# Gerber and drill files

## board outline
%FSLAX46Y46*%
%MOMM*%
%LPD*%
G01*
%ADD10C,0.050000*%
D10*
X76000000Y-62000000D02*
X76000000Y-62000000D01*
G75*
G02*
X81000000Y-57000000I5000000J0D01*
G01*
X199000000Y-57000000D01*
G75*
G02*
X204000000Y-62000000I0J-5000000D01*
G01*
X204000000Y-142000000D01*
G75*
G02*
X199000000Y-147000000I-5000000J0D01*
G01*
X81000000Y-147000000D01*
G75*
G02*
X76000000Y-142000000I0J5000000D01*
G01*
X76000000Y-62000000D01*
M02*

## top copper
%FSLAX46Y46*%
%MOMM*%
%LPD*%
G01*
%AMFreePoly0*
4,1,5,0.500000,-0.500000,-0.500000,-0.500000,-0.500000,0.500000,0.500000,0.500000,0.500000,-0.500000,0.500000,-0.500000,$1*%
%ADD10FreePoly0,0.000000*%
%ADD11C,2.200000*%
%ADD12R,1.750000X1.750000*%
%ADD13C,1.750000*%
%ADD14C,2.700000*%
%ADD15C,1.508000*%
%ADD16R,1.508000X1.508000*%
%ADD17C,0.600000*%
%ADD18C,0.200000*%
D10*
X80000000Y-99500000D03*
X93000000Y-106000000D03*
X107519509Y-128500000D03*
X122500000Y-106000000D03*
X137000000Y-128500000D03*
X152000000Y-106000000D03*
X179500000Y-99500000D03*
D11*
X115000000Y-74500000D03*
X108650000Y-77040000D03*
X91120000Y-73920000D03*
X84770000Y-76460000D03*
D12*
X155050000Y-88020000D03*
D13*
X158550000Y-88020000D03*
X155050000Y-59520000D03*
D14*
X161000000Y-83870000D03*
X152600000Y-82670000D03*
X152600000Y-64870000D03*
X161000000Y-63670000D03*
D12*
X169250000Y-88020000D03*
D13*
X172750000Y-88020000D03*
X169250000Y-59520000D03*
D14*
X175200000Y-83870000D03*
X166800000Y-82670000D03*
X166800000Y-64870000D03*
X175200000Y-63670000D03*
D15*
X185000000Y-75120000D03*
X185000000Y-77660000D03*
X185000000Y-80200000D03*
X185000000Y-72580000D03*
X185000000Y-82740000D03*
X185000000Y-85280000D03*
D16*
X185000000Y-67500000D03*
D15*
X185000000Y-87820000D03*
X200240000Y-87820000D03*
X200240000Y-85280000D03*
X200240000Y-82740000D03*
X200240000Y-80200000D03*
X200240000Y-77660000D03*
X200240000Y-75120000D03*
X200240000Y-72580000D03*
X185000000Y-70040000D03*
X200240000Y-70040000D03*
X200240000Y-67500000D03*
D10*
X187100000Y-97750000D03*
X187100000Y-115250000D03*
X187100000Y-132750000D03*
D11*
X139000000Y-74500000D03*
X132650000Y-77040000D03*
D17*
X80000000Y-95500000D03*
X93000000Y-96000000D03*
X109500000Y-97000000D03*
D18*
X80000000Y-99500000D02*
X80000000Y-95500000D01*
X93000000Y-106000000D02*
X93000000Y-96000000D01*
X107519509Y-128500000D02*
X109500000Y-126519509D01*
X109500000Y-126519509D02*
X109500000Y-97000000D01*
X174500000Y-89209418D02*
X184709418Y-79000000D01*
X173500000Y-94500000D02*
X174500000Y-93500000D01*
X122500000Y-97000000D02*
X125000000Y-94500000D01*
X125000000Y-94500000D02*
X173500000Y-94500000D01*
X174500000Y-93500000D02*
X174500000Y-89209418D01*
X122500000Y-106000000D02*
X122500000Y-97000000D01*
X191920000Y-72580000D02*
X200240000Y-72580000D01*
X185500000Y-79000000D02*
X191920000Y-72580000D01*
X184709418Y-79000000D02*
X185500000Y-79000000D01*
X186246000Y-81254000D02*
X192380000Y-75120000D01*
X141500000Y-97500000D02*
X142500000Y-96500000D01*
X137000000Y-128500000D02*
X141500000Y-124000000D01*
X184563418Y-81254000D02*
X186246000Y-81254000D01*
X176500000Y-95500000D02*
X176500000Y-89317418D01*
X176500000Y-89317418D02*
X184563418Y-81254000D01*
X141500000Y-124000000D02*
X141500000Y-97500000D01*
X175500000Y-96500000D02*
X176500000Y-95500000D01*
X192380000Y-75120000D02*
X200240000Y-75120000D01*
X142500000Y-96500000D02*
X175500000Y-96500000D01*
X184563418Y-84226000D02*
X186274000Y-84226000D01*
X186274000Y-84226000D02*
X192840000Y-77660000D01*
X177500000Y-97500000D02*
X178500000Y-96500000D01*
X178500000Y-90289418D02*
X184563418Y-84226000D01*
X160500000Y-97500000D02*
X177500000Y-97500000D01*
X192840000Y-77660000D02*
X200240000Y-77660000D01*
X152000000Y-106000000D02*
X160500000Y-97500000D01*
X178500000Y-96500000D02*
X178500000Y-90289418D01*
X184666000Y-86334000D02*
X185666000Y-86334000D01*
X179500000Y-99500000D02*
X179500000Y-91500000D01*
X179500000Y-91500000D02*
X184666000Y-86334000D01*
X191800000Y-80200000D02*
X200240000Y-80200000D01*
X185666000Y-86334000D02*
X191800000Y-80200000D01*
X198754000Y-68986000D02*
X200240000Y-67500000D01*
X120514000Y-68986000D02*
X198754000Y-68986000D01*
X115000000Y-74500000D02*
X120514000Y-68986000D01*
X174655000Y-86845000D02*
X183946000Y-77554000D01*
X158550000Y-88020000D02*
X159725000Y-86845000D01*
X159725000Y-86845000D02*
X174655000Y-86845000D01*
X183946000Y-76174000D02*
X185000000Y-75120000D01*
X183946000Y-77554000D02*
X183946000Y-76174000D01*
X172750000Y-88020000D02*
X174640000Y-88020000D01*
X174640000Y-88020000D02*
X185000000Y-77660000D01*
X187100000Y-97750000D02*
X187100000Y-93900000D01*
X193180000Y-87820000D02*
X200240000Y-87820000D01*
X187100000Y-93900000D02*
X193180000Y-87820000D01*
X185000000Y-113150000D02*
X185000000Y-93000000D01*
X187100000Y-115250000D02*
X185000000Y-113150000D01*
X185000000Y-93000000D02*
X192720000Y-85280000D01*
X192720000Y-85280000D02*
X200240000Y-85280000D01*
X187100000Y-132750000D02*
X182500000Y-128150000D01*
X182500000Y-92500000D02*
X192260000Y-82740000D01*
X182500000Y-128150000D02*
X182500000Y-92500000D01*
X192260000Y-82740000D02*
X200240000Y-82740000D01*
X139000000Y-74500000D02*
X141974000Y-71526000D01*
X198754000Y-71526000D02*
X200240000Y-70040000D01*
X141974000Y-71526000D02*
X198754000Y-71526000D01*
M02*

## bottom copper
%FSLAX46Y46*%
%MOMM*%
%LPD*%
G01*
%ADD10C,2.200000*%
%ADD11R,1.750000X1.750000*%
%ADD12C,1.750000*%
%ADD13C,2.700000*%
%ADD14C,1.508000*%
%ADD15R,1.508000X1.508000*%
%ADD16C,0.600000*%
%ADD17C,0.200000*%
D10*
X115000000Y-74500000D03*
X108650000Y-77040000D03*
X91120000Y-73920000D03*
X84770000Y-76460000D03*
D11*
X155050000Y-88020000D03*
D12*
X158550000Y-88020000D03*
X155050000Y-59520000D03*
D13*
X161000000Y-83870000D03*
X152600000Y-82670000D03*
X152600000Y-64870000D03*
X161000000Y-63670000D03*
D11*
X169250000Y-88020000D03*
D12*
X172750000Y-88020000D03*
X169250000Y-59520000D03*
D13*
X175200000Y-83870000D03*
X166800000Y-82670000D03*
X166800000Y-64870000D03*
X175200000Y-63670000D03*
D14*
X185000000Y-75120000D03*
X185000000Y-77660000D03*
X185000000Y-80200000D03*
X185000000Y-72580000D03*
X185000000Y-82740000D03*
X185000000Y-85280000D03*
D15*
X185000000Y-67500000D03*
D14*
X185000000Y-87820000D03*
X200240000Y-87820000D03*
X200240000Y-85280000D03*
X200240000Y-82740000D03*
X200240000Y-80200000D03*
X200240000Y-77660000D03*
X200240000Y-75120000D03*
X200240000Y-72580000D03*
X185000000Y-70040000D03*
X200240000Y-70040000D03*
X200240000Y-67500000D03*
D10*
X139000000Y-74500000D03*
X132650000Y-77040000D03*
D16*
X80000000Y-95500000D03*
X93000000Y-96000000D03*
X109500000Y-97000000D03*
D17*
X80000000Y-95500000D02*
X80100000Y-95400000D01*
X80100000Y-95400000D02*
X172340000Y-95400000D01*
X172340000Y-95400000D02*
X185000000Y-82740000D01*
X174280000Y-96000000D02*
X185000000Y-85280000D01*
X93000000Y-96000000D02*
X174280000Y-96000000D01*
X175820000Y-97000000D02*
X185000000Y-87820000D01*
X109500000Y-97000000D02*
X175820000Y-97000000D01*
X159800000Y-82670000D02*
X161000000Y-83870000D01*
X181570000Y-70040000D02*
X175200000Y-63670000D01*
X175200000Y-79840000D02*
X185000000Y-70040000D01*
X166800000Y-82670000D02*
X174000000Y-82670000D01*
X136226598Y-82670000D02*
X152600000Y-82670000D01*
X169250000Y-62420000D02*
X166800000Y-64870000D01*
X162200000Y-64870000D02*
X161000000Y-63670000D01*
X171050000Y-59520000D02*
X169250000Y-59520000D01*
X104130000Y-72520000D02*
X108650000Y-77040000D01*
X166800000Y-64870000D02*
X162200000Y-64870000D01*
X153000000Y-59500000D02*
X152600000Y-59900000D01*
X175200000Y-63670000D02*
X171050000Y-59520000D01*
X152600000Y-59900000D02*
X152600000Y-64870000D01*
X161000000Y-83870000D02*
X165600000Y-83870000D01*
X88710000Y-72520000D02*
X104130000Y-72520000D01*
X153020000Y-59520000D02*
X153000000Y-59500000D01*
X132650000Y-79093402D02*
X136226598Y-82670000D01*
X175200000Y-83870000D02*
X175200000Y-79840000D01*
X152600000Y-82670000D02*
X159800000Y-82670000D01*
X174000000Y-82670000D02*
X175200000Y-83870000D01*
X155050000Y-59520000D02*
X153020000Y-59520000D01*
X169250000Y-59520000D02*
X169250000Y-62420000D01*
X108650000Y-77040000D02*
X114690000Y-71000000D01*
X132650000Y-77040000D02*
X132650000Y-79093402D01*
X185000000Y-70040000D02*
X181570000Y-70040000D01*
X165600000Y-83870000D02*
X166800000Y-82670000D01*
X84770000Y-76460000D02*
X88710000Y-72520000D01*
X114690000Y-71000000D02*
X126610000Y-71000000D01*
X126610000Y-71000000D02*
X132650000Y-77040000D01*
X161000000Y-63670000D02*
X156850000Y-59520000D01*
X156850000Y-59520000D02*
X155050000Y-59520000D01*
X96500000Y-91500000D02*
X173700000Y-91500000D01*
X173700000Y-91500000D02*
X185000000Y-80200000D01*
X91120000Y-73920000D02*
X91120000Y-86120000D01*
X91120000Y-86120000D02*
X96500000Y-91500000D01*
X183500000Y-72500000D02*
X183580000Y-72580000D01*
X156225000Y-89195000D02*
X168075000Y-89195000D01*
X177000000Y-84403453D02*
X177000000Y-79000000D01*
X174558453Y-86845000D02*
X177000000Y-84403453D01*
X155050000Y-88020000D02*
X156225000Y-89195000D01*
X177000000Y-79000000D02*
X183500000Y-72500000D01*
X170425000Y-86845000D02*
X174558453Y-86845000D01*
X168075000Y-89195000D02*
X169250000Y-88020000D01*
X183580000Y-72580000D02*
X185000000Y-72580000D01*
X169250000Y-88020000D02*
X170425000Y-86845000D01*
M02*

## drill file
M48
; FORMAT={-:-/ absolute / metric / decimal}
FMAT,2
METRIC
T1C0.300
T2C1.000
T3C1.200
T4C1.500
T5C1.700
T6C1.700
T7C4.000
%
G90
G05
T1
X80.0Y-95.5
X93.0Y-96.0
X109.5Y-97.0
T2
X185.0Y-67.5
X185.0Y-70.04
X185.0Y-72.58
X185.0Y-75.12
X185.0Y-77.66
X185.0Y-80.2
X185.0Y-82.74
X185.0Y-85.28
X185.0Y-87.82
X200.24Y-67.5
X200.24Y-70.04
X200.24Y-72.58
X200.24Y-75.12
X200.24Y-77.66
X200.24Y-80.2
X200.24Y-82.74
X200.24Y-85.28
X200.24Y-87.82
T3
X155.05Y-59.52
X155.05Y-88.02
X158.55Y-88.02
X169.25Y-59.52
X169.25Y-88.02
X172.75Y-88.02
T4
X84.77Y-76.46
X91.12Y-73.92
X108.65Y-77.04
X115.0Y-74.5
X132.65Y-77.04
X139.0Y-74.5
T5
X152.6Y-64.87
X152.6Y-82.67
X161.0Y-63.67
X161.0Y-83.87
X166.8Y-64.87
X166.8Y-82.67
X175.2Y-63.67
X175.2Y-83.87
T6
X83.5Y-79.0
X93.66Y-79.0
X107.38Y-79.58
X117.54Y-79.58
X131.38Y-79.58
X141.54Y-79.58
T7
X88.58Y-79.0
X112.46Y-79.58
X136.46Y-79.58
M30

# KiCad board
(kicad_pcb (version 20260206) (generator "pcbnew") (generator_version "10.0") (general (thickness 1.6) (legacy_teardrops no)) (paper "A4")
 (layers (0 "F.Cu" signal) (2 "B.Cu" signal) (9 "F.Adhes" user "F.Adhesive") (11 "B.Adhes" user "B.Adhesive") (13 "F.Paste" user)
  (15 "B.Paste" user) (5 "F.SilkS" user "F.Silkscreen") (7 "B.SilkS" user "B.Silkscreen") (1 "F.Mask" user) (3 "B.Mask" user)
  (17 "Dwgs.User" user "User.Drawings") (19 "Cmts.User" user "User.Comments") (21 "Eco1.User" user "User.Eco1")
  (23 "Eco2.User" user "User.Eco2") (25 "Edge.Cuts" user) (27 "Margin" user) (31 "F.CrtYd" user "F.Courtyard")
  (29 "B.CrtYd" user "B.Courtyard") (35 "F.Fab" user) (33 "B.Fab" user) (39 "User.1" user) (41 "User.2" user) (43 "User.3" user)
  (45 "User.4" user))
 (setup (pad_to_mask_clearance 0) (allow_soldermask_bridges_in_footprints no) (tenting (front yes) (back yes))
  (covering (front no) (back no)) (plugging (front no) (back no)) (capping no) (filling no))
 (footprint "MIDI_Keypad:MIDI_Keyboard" (layer "F.Cu") (at 104 43)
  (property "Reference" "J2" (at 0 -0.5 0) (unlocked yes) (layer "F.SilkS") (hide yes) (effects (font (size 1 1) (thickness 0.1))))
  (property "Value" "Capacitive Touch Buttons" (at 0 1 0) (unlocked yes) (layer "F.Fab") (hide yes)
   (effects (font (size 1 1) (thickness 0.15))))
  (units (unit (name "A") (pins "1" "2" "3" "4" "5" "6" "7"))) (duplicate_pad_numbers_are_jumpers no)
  (pad "1" smd custom (at -24 56.5) (size 1 1) (layers "F.Cu" "F.Mask") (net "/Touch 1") (options (clearance outline) (anchor rect))
   (primitives))
  (pad "2" smd custom (at -11 63) (size 1 1) (layers "F.Cu" "F.Mask") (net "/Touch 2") (options (clearance outline) (anchor rect))
   (primitives))
  (pad "3" smd custom (at 3.519509 85.5) (size 1 1) (layers "F.Cu" "F.Mask") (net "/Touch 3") (options (clearance outline) (anchor rect))
   (primitives))
  (pad "4" smd custom (at 18.5 63) (size 1 1) (layers "F.Cu" "F.Mask") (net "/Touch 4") (options (clearance outline) (anchor rect))
   (primitives))
  (pad "5" smd custom (at 33 85.5) (size 1 1) (layers "F.Cu" "F.Mask") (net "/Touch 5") (options (clearance outline) (anchor rect))
   (primitives))
  (pad "6" smd custom (at 48 63) (size 1 1) (layers "F.Cu" "F.Mask") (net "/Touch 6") (options (clearance outline) (anchor rect))
   (primitives))
  (pad "7" smd custom (at 75.5 56.5) (size 1 1) (layers "F.Cu" "F.Mask") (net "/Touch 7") (options (clearance outline) (anchor rect))
   (primitives)))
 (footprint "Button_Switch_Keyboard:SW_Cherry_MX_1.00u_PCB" (layer "F.Cu") (at 115 74.5)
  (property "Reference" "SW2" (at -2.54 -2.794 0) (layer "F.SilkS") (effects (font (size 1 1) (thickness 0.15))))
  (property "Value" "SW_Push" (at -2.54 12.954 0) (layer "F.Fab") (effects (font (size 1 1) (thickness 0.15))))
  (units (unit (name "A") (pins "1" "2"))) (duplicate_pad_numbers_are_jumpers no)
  (pad "" np_thru_hole circle (at -7.62 5.08) (size 1.7 1.7) (drill 1.7) (layers "*.Cu" "*.Mask"))
  (pad "" np_thru_hole circle (at -2.54 5.08) (size 4 4) (drill 4) (layers "*.Cu" "*.Mask"))
  (pad "" np_thru_hole circle (at 2.54 5.08) (size 1.7 1.7) (drill 1.7) (layers "*.Cu" "*.Mask"))
  (pad "1" thru_hole circle (at 0 0) (size 2.2 2.2) (drill 1.5) (layers "*.Cu" "*.Mask") (remove_unused_layers no) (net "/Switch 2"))
  (pad "2" thru_hole circle (at -6.35 2.54) (size 2.2 2.2) (drill 1.5) (layers "*.Cu" "*.Mask") (remove_unused_layers no) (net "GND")))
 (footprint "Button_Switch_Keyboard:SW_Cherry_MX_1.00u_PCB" (layer "F.Cu") (at 91.12 73.92)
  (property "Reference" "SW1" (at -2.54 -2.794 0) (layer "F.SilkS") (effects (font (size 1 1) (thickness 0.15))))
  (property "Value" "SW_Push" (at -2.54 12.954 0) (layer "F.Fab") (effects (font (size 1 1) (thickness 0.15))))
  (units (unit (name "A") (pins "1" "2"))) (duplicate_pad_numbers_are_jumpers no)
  (pad "" np_thru_hole circle (at -7.62 5.08) (size 1.7 1.7) (drill 1.7) (layers "*.Cu" "*.Mask"))
  (pad "" np_thru_hole circle (at -2.54 5.08) (size 4 4) (drill 4) (layers "*.Cu" "*.Mask"))
  (pad "" np_thru_hole circle (at 2.54 5.08) (size 1.7 1.7) (drill 1.7) (layers "*.Cu" "*.Mask"))
  (pad "1" thru_hole circle (at 0 0) (size 2.2 2.2) (drill 1.5) (layers "*.Cu" "*.Mask") (remove_unused_layers no) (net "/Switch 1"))
  (pad "2" thru_hole circle (at -6.35 2.54) (size 2.2 2.2) (drill 1.5) (layers "*.Cu" "*.Mask") (remove_unused_layers no) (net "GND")))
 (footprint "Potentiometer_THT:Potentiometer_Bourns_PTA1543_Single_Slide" (layer "F.Cu") (at 155.05 88.02 90)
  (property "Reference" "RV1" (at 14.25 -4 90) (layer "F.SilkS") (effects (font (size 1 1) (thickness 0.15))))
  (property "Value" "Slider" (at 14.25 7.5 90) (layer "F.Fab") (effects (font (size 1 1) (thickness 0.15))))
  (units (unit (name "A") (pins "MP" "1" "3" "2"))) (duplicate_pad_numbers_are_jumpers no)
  (pad "1" thru_hole rect (at 0 0 90) (size 1.75 1.75) (drill 1.2) (layers "*.Cu" "*.Mask") (remove_unused_layers no) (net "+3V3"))
  (pad "2" thru_hole circle (at 0 3.5 90) (size 1.75 1.75) (drill 1.2) (layers "*.Cu" "*.Mask") (remove_unused_layers no) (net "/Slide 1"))
  (pad "3" thru_hole circle (at 28.5 0 90) (size 1.75 1.75) (drill 1.2) (layers "*.Cu" "*.Mask") (remove_unused_layers no) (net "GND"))
  (pad "MP" thru_hole circle (at 4.15 5.95 90) (size 2.7 2.7) (drill 1.7) (layers "*.Cu" "*.Mask") (remove_unused_layers no) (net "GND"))
  (pad "MP" thru_hole circle (at 5.35 -2.45 90) (size 2.7 2.7) (drill 1.7) (layers "*.Cu" "*.Mask") (remove_unused_layers no) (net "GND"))
  (pad "MP" thru_hole circle (at 23.15 -2.45 90) (size 2.7 2.7) (drill 1.7) (layers "*.Cu" "*.Mask") (remove_unused_layers no) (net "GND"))
  (pad "MP" thru_hole circle (at 24.35 5.95 90) (size 2.7 2.7) (drill 1.7) (layers "*.Cu" "*.Mask") (remove_unused_layers no) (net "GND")))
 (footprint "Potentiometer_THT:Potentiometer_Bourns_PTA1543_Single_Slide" (layer "F.Cu") (at 169.25 88.02 90)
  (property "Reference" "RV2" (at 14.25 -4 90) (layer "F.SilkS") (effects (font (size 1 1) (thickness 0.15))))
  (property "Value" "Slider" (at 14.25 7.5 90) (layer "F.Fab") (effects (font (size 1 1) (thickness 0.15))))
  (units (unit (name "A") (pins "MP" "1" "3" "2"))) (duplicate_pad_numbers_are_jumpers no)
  (pad "1" thru_hole rect (at 0 0 90) (size 1.75 1.75) (drill 1.2) (layers "*.Cu" "*.Mask") (remove_unused_layers no) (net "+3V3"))
  (pad "2" thru_hole circle (at 0 3.5 90) (size 1.75 1.75) (drill 1.2) (layers "*.Cu" "*.Mask") (remove_unused_layers no) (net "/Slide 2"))
  (pad "3" thru_hole circle (at 28.5 0 90) (size 1.75 1.75) (drill 1.2) (layers "*.Cu" "*.Mask") (remove_unused_layers no) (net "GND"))
  (pad "MP" thru_hole circle (at 4.15 5.95 90) (size 2.7 2.7) (drill 1.7) (layers "*.Cu" "*.Mask") (remove_unused_layers no) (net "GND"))
  (pad "MP" thru_hole circle (at 5.35 -2.45 90) (size 2.7 2.7) (drill 1.7) (layers "*.Cu" "*.Mask") (remove_unused_layers no) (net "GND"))
  (pad "MP" thru_hole circle (at 23.15 -2.45 90) (size 2.7 2.7) (drill 1.7) (layers "*.Cu" "*.Mask") (remove_unused_layers no) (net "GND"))
  (pad "MP" thru_hole circle (at 24.35 5.95 90) (size 2.7 2.7) (drill 1.7) (layers "*.Cu" "*.Mask") (remove_unused_layers no) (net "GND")))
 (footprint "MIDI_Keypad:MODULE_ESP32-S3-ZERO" (layer "F.Cu") (at 192.62 77.66)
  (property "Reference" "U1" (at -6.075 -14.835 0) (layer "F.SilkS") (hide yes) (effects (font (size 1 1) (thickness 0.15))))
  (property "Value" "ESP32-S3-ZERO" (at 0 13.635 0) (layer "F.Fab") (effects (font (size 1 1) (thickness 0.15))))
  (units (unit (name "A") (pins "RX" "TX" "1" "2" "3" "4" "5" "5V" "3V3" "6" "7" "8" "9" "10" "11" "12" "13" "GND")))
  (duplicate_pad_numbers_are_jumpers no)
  (pad "1" thru_hole circle (at -7.62 -2.54) (size 1.508 1.508) (drill 1) (layers "*.Cu" "*.Mask") (remove_unused_layers no)
   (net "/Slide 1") (solder_mask_margin 0.102))
  (pad "2" thru_hole circle (at -7.62 0) (size 1.508 1.508) (drill 1) (layers "*.Cu" "*.Mask") (remove_unused_layers no) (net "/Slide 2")
   (solder_mask_margin 0.102))
  (pad "3" thru_hole circle (at -7.62 2.54) (size 1.508 1.508) (drill 1) (layers "*.Cu" "*.Mask") (remove_unused_layers no)
   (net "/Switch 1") (solder_mask_margin 0.102))
  (pad "3V3" thru_hole circle (at -7.62 -5.08) (size 1.508 1.508) (drill 1) (layers "*.Cu" "*.Mask") (remove_unused_layers no) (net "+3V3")
   (solder_mask_margin 0.102))
  (pad "4" thru_hole circle (at -7.62 5.08) (size 1.508 1.508) (drill 1) (layers "*.Cu" "*.Mask") (remove_unused_layers no) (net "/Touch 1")
   (solder_mask_margin 0.102))
  (pad "5" thru_hole circle (at -7.62 7.62) (size 1.508 1.508) (drill 1) (layers "*.Cu" "*.Mask") (remove_unused_layers no) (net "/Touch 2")
   (solder_mask_margin 0.102))
  (pad "5V" thru_hole rect (at -7.62 -10.16) (size 1.508 1.508) (drill 1) (layers "*.Cu" "*.Mask") (remove_unused_layers no) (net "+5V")
   (solder_mask_margin 0.102))
  (pad "6" thru_hole circle (at -7.62 10.16) (size 1.508 1.508) (drill 1) (layers "*.Cu" "*.Mask") (remove_unused_layers no)
   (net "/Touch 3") (solder_mask_margin 0.102))
  (pad "7" thru_hole circle (at 7.62 10.16) (size 1.508 1.508) (drill 1) (layers "*.Cu" "*.Mask") (remove_unused_layers no) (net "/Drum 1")
   (solder_mask_margin 0.102))
  (pad "8" thru_hole circle (at 7.62 7.62) (size 1.508 1.508) (drill 1) (layers "*.Cu" "*.Mask") (remove_unused_layers no) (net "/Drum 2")
   (solder_mask_margin 0.102))
  (pad "9" thru_hole circle (at 7.62 5.08) (size 1.508 1.508) (drill 1) (layers "*.Cu" "*.Mask") (remove_unused_layers no) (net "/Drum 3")
   (solder_mask_margin 0.102))
  (pad "10" thru_hole circle (at 7.62 2.54) (size 1.508 1.508) (drill 1) (layers "*.Cu" "*.Mask") (remove_unused_layers no) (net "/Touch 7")
   (solder_mask_margin 0.102))
  (pad "11" thru_hole circle (at 7.62 0) (size 1.508 1.508) (drill 1) (layers "*.Cu" "*.Mask") (remove_unused_layers no) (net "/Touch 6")
   (solder_mask_margin 0.102))
  (pad "12" thru_hole circle (at 7.62 -2.54) (size 1.508 1.508) (drill 1) (layers "*.Cu" "*.Mask") (remove_unused_layers no)
   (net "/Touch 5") (solder_mask_margin 0.102))
  (pad "13" thru_hole circle (at 7.62 -5.08) (size 1.508 1.508) (drill 1) (layers "*.Cu" "*.Mask") (remove_unused_layers no)
   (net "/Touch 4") (solder_mask_margin 0.102))
  (pad "GND" thru_hole circle (at -7.62 -7.62) (size 1.508 1.508) (drill 1) (layers "*.Cu" "*.Mask") (remove_unused_layers no) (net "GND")
   (solder_mask_margin 0.102))
  (pad "RX" thru_hole circle (at 7.62 -7.62) (size 1.508 1.508) (drill 1) (layers "*.Cu" "*.Mask") (remove_unused_layers no)
   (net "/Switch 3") (solder_mask_margin 0.102))
  (pad "TX" thru_hole circle (at 7.62 -10.16) (size 1.508 1.508) (drill 1) (layers "*.Cu" "*.Mask") (remove_unused_layers no)
   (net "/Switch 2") (solder_mask_margin 0.102)))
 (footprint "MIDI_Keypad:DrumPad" (layer "F.Cu") (at 191.1 90.75)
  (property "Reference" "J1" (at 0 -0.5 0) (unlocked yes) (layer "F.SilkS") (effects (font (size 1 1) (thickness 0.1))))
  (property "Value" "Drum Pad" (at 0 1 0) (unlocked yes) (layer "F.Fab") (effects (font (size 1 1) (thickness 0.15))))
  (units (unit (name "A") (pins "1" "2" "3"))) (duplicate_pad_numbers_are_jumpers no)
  (pad "1" smd custom (at -4 7) (size 1 1) (layers "F.Cu" "F.Mask") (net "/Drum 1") (options (clearance outline) (anchor rect)) (primitives))
  (pad "2" smd custom (at -4 24.5) (size 1 1) (layers "F.Cu" "F.Mask") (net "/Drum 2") (options (clearance outline) (anchor rect))
   (primitives))
  (pad "3" smd custom (at -4 42) (size 1 1) (layers "F.Cu" "F.Mask") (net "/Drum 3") (options (clearance outline) (anchor rect))
   (primitives)))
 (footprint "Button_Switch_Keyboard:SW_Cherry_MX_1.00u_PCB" (layer "F.Cu") (at 139 74.5)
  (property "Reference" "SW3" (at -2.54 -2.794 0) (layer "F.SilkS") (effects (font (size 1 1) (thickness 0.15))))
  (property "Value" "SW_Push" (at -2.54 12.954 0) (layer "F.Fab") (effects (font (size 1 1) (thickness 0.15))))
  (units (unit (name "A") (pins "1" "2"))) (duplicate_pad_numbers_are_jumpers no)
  (pad "" np_thru_hole circle (at -7.62 5.08) (size 1.7 1.7) (drill 1.7) (layers "*.Cu" "*.Mask"))
  (pad "" np_thru_hole circle (at -2.54 5.08) (size 4 4) (drill 4) (layers "*.Cu" "*.Mask"))
  (pad "" np_thru_hole circle (at 2.54 5.08) (size 1.7 1.7) (drill 1.7) (layers "*.Cu" "*.Mask"))
  (pad "1" thru_hole circle (at 0 0) (size 2.2 2.2) (drill 1.5) (layers "*.Cu" "*.Mask") (remove_unused_layers no) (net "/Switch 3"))
  (pad "2" thru_hole circle (at -6.35 2.54) (size 2.2 2.2) (drill 1.5) (layers "*.Cu" "*.Mask") (remove_unused_layers no) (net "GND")))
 (gr_rect (start 76 57) (end 204 147) (radius 5) (stroke (width 0.05) (type solid)) (fill no) (layer "Edge.Cuts"))
 (segment (start 80 99.5) (end 80 95.5) (width 0.2) (layer "F.Cu") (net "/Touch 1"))
 (via (at 80 95.5) (size 0.6) (drill 0.3) (layers "F.Cu" "B.Cu") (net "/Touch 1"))
 (segment (start 80 95.5) (end 80.1 95.4) (width 0.2) (layer "B.Cu") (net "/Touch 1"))
 (segment (start 80.1 95.4) (end 172.34 95.4) (width 0.2) (layer "B.Cu") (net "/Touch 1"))
 (segment (start 172.34 95.4) (end 185 82.74) (width 0.2) (layer "B.Cu") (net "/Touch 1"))
 (segment (start 93 106) (end 93 96) (width 0.2) (layer "F.Cu") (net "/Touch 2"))
 (via (at 93 96) (size 0.6) (drill 0.3) (layers "F.Cu" "B.Cu") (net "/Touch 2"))
 (segment (start 174.28 96) (end 185 85.28) (width 0.2) (layer "B.Cu") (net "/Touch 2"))
 (segment (start 93 96) (end 174.28 96) (width 0.2) (layer "B.Cu") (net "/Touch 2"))
 (segment (start 107.519509 128.5) (end 109.5 126.519509) (width 0.2) (layer "F.Cu") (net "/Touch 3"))
 (segment (start 109.5 126.519509) (end 109.5 97) (width 0.2) (layer "F.Cu") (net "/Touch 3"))
 (via (at 109.5 97) (size 0.6) (drill 0.3) (layers "F.Cu" "B.Cu") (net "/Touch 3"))
 (segment (start 175.82 97) (end 185 87.82) (width 0.2) (layer "B.Cu") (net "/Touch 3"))
 (segment (start 109.5 97) (end 175.82 97) (width 0.2) (layer "B.Cu") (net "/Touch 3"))
 (segment (start 174.5 89.209418) (end 184.709418 79) (width 0.2) (layer "F.Cu") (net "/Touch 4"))
 (segment (start 173.5 94.5) (end 174.5 93.5) (width 0.2) (layer "F.Cu") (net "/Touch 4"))
 (segment (start 122.5 97) (end 125 94.5) (width 0.2) (layer "F.Cu") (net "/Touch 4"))
 (segment (start 125 94.5) (end 173.5 94.5) (width 0.2) (layer "F.Cu") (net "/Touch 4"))
 (segment (start 174.5 93.5) (end 174.5 89.209418) (width 0.2) (layer "F.Cu") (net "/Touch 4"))
 (segment (start 122.5 106) (end 122.5 97) (width 0.2) (layer "F.Cu") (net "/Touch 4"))
 (segment (start 191.92 72.58) (end 200.24 72.58) (width 0.2) (layer "F.Cu") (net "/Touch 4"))
 (segment (start 185.5 79) (end 191.92 72.58) (width 0.2) (layer "F.Cu") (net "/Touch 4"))
 (segment (start 184.709418 79) (end 185.5 79) (width 0.2) (layer "F.Cu") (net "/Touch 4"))
 (segment (start 186.246 81.254) (end 192.38 75.12) (width 0.2) (layer "F.Cu") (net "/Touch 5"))
 (segment (start 141.5 97.5) (end 142.5 96.5) (width 0.2) (layer "F.Cu") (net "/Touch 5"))
 (segment (start 137 128.5) (end 141.5 124) (width 0.2) (layer "F.Cu") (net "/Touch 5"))
 (segment (start 184.563418 81.254) (end 186.246 81.254) (width 0.2) (layer "F.Cu") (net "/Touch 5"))
 (segment (start 176.5 95.5) (end 176.5 89.317418) (width 0.2) (layer "F.Cu") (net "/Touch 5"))
 (segment (start 176.5 89.317418) (end 184.563418 81.254) (width 0.2) (layer "F.Cu") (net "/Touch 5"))
 (segment (start 141.5 124) (end 141.5 97.5) (width 0.2) (layer "F.Cu") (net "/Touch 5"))
 (segment (start 175.5 96.5) (end 176.5 95.5) (width 0.2) (layer "F.Cu") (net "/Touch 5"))
 (segment (start 192.38 75.12) (end 200.24 75.12) (width 0.2) (layer "F.Cu") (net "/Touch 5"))
 (segment (start 142.5 96.5) (end 175.5 96.5) (width 0.2) (layer "F.Cu") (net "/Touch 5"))
 (segment (start 184.563418 84.226) (end 186.274 84.226) (width 0.2) (layer "F.Cu") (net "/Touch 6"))
 (segment (start 186.274 84.226) (end 192.84 77.66) (width 0.2) (layer "F.Cu") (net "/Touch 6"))
 (segment (start 177.5 97.5) (end 178.5 96.5) (width 0.2) (layer "F.Cu") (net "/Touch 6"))
 (segment (start 178.5 90.289418) (end 184.563418 84.226) (width 0.2) (layer "F.Cu") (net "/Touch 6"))
 (segment (start 160.5 97.5) (end 177.5 97.5) (width 0.2) (layer "F.Cu") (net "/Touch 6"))
 (segment (start 192.84 77.66) (end 200.24 77.66) (width 0.2) (layer "F.Cu") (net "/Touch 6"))
 (segment (start 152 106) (end 160.5 97.5) (width 0.2) (layer "F.Cu") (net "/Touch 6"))
 (segment (start 178.5 96.5) (end 178.5 90.289418) (width 0.2) (layer "F.Cu") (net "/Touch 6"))
 (segment (start 184.666 86.334) (end 185.666 86.334) (width 0.2) (layer "F.Cu") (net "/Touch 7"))
 (segment (start 179.5 99.5) (end 179.5 91.5) (width 0.2) (layer "F.Cu") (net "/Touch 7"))
 (segment (start 179.5 91.5) (end 184.666 86.334) (width 0.2) (layer "F.Cu") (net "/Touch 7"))
 (segment (start 191.8 80.2) (end 200.24 80.2) (width 0.2) (layer "F.Cu") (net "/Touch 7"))
 (segment (start 185.666 86.334) (end 191.8 80.2) (width 0.2) (layer "F.Cu") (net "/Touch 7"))
 (segment (start 198.754 68.986) (end 200.24 67.5) (width 0.2) (layer "F.Cu") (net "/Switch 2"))
 (segment (start 120.514 68.986) (end 198.754 68.986) (width 0.2) (layer "F.Cu") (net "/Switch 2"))
 (segment (start 115 74.5) (end 120.514 68.986) (width 0.2) (layer "F.Cu") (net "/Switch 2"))
 (segment (start 159.8 82.67) (end 161 83.87) (width 0.2) (layer "B.Cu") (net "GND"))
 (segment (start 181.57 70.04) (end 175.2 63.67) (width 0.2) (layer "B.Cu") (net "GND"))
 (segment (start 175.2 79.84) (end 185 70.04) (width 0.2) (layer "B.Cu") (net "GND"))
 (segment (start 166.8 82.67) (end 174 82.67) (width 0.2) (layer "B.Cu") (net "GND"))
 (segment (start 136.226598 82.67) (end 152.6 82.67) (width 0.2) (layer "B.Cu") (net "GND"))
 (segment (start 169.25 62.42) (end 166.8 64.87) (width 0.2) (layer "B.Cu") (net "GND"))
 (segment (start 162.2 64.87) (end 161 63.67) (width 0.2) (layer "B.Cu") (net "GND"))
 (segment (start 171.05 59.52) (end 169.25 59.52) (width 0.2) (layer "B.Cu") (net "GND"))
 (segment (start 104.13 72.52) (end 108.65 77.04) (width 0.2) (layer "B.Cu") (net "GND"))
 (segment (start 166.8 64.87) (end 162.2 64.87) (width 0.2) (layer "B.Cu") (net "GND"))
 (segment (start 153 59.5) (end 152.6 59.9) (width 0.2) (layer "B.Cu") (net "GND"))
 (segment (start 175.2 63.67) (end 171.05 59.52) (width 0.2) (layer "B.Cu") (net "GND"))
 (segment (start 152.6 59.9) (end 152.6 64.87) (width 0.2) (layer "B.Cu") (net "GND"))
 (segment (start 161 83.87) (end 165.6 83.87) (width 0.2) (layer "B.Cu") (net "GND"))
 (segment (start 88.71 72.52) (end 104.13 72.52) (width 0.2) (layer "B.Cu") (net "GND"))
 (segment (start 153.02 59.52) (end 153 59.5) (width 0.2) (layer "B.Cu") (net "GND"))
 (segment (start 132.65 79.093402) (end 136.226598 82.67) (width 0.2) (layer "B.Cu") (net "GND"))
 (segment (start 175.2 83.87) (end 175.2 79.84) (width 0.2) (layer "B.Cu") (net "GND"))
 (segment (start 152.6 82.67) (end 159.8 82.67) (width 0.2) (layer "B.Cu") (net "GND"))
 (segment (start 174 82.67) (end 175.2 83.87) (width 0.2) (layer "B.Cu") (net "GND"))
 (segment (start 155.05 59.52) (end 153.02 59.52) (width 0.2) (layer "B.Cu") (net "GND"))
 (segment (start 169.25 59.52) (end 169.25 62.42) (width 0.2) (layer "B.Cu") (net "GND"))
 (segment (start 108.65 77.04) (end 114.69 71) (width 0.2) (layer "B.Cu") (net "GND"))
 (segment (start 132.65 77.04) (end 132.65 79.093402) (width 0.2) (layer "B.Cu") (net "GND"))
 (segment (start 185 70.04) (end 181.57 70.04) (width 0.2) (layer "B.Cu") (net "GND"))
 (segment (start 165.6 83.87) (end 166.8 82.67) (width 0.2) (layer "B.Cu") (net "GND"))
 (segment (start 84.77 76.46) (end 88.71 72.52) (width 0.2) (layer "B.Cu") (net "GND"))
 (segment (start 114.69 71) (end 126.61 71) (width 0.2) (layer "B.Cu") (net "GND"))
 (segment (start 126.61 71) (end 132.65 77.04) (width 0.2) (layer "B.Cu") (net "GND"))
 (segment (start 161 63.67) (end 156.85 59.52) (width 0.2) (layer "B.Cu") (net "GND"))
 (segment (start 156.85 59.52) (end 155.05 59.52) (width 0.2) (layer "B.Cu") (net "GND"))
 (segment (start 96.5 91.5) (end 173.7 91.5) (width 0.2) (layer "B.Cu") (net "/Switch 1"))
 (segment (start 173.7 91.5) (end 185 80.2) (width 0.2) (layer "B.Cu") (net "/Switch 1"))
 (segment (start 91.12 73.92) (end 91.12 86.12) (width 0.2) (layer "B.Cu") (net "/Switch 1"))
 (segment (start 91.12 86.12) (end 96.5 91.5) (width 0.2) (layer "B.Cu") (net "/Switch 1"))
 (segment (start 183.5 72.5) (end 183.58 72.58) (width 0.2) (layer "B.Cu") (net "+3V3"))
 (segment (start 156.225 89.195) (end 168.075 89.195) (width 0.2) (layer "B.Cu") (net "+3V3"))
 (segment (start 177 84.403453) (end 177 79) (width 0.2) (layer "B.Cu") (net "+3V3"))
 (segment (start 174.558453 86.845) (end 177 84.403453) (width 0.2) (layer "B.Cu") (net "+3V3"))
 (segment (start 155.05 88.02) (end 156.225 89.195) (width 0.2) (layer "B.Cu") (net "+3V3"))
 (segment (start 177 79) (end 183.5 72.5) (width 0.2) (layer "B.Cu") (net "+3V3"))
 (segment (start 170.425 86.845) (end 174.558453 86.845) (width 0.2) (layer "B.Cu") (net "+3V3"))
 (segment (start 168.075 89.195) (end 169.25 88.02) (width 0.2) (layer "B.Cu") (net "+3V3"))
 (segment (start 183.58 72.58) (end 185 72.58) (width 0.2) (layer "B.Cu") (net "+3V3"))
 (segment (start 169.25 88.02) (end 170.425 86.845) (width 0.2) (layer "B.Cu") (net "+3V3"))
 (segment (start 174.655 86.845) (end 183.946 77.554) (width 0.2) (layer "F.Cu") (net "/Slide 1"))
 (segment (start 158.55 88.02) (end 159.725 86.845) (width 0.2) (layer "F.Cu") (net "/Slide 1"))
 (segment (start 159.725 86.845) (end 174.655 86.845) (width 0.2) (layer "F.Cu") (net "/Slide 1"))
 (segment (start 183.946 76.174) (end 185 75.12) (width 0.2) (layer "F.Cu") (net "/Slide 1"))
 (segment (start 183.946 77.554) (end 183.946 76.174) (width 0.2) (layer "F.Cu") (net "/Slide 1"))
 (segment (start 172.75 88.02) (end 174.64 88.02) (width 0.2) (layer "F.Cu") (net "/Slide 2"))
 (segment (start 174.64 88.02) (end 185 77.66) (width 0.2) (layer "F.Cu") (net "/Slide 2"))
 (segment (start 187.1 97.75) (end 187.1 93.9) (width 0.2) (layer "F.Cu") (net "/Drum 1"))
 (segment (start 193.18 87.82) (end 200.24 87.82) (width 0.2) (layer "F.Cu") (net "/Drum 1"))
 (segment (start 187.1 93.9) (end 193.18 87.82) (width 0.2) (layer "F.Cu") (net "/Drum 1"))
 (segment (start 185 113.15) (end 185 93) (width 0.2) (layer "F.Cu") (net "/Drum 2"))
 (segment (start 187.1 115.25) (end 185 113.15) (width 0.2) (layer "F.Cu") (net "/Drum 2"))
 (segment (start 185 93) (end 192.72 85.28) (width 0.2) (layer "F.Cu") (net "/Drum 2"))
 (segment (start 192.72 85.28) (end 200.24 85.28) (width 0.2) (layer "F.Cu") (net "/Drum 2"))
 (segment (start 187.1 132.75) (end 182.5 128.15) (width 0.2) (layer "F.Cu") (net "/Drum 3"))
 (segment (start 182.5 92.5) (end 192.26 82.74) (width 0.2) (layer "F.Cu") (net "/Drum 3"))
 (segment (start 182.5 128.15) (end 182.5 92.5) (width 0.2) (layer "F.Cu") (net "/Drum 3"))
 (segment (start 192.26 82.74) (end 200.24 82.74) (width 0.2) (layer "F.Cu") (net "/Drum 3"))
 (segment (start 139 74.5) (end 141.974 71.526) (width 0.2) (layer "F.Cu") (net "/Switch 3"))
 (segment (start 198.754 71.526) (end 200.24 70.04) (width 0.2) (layer "F.Cu") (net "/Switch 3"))
 (segment (start 141.974 71.526) (end 198.754 71.526) (width 0.2) (layer "F.Cu") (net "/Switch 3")))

